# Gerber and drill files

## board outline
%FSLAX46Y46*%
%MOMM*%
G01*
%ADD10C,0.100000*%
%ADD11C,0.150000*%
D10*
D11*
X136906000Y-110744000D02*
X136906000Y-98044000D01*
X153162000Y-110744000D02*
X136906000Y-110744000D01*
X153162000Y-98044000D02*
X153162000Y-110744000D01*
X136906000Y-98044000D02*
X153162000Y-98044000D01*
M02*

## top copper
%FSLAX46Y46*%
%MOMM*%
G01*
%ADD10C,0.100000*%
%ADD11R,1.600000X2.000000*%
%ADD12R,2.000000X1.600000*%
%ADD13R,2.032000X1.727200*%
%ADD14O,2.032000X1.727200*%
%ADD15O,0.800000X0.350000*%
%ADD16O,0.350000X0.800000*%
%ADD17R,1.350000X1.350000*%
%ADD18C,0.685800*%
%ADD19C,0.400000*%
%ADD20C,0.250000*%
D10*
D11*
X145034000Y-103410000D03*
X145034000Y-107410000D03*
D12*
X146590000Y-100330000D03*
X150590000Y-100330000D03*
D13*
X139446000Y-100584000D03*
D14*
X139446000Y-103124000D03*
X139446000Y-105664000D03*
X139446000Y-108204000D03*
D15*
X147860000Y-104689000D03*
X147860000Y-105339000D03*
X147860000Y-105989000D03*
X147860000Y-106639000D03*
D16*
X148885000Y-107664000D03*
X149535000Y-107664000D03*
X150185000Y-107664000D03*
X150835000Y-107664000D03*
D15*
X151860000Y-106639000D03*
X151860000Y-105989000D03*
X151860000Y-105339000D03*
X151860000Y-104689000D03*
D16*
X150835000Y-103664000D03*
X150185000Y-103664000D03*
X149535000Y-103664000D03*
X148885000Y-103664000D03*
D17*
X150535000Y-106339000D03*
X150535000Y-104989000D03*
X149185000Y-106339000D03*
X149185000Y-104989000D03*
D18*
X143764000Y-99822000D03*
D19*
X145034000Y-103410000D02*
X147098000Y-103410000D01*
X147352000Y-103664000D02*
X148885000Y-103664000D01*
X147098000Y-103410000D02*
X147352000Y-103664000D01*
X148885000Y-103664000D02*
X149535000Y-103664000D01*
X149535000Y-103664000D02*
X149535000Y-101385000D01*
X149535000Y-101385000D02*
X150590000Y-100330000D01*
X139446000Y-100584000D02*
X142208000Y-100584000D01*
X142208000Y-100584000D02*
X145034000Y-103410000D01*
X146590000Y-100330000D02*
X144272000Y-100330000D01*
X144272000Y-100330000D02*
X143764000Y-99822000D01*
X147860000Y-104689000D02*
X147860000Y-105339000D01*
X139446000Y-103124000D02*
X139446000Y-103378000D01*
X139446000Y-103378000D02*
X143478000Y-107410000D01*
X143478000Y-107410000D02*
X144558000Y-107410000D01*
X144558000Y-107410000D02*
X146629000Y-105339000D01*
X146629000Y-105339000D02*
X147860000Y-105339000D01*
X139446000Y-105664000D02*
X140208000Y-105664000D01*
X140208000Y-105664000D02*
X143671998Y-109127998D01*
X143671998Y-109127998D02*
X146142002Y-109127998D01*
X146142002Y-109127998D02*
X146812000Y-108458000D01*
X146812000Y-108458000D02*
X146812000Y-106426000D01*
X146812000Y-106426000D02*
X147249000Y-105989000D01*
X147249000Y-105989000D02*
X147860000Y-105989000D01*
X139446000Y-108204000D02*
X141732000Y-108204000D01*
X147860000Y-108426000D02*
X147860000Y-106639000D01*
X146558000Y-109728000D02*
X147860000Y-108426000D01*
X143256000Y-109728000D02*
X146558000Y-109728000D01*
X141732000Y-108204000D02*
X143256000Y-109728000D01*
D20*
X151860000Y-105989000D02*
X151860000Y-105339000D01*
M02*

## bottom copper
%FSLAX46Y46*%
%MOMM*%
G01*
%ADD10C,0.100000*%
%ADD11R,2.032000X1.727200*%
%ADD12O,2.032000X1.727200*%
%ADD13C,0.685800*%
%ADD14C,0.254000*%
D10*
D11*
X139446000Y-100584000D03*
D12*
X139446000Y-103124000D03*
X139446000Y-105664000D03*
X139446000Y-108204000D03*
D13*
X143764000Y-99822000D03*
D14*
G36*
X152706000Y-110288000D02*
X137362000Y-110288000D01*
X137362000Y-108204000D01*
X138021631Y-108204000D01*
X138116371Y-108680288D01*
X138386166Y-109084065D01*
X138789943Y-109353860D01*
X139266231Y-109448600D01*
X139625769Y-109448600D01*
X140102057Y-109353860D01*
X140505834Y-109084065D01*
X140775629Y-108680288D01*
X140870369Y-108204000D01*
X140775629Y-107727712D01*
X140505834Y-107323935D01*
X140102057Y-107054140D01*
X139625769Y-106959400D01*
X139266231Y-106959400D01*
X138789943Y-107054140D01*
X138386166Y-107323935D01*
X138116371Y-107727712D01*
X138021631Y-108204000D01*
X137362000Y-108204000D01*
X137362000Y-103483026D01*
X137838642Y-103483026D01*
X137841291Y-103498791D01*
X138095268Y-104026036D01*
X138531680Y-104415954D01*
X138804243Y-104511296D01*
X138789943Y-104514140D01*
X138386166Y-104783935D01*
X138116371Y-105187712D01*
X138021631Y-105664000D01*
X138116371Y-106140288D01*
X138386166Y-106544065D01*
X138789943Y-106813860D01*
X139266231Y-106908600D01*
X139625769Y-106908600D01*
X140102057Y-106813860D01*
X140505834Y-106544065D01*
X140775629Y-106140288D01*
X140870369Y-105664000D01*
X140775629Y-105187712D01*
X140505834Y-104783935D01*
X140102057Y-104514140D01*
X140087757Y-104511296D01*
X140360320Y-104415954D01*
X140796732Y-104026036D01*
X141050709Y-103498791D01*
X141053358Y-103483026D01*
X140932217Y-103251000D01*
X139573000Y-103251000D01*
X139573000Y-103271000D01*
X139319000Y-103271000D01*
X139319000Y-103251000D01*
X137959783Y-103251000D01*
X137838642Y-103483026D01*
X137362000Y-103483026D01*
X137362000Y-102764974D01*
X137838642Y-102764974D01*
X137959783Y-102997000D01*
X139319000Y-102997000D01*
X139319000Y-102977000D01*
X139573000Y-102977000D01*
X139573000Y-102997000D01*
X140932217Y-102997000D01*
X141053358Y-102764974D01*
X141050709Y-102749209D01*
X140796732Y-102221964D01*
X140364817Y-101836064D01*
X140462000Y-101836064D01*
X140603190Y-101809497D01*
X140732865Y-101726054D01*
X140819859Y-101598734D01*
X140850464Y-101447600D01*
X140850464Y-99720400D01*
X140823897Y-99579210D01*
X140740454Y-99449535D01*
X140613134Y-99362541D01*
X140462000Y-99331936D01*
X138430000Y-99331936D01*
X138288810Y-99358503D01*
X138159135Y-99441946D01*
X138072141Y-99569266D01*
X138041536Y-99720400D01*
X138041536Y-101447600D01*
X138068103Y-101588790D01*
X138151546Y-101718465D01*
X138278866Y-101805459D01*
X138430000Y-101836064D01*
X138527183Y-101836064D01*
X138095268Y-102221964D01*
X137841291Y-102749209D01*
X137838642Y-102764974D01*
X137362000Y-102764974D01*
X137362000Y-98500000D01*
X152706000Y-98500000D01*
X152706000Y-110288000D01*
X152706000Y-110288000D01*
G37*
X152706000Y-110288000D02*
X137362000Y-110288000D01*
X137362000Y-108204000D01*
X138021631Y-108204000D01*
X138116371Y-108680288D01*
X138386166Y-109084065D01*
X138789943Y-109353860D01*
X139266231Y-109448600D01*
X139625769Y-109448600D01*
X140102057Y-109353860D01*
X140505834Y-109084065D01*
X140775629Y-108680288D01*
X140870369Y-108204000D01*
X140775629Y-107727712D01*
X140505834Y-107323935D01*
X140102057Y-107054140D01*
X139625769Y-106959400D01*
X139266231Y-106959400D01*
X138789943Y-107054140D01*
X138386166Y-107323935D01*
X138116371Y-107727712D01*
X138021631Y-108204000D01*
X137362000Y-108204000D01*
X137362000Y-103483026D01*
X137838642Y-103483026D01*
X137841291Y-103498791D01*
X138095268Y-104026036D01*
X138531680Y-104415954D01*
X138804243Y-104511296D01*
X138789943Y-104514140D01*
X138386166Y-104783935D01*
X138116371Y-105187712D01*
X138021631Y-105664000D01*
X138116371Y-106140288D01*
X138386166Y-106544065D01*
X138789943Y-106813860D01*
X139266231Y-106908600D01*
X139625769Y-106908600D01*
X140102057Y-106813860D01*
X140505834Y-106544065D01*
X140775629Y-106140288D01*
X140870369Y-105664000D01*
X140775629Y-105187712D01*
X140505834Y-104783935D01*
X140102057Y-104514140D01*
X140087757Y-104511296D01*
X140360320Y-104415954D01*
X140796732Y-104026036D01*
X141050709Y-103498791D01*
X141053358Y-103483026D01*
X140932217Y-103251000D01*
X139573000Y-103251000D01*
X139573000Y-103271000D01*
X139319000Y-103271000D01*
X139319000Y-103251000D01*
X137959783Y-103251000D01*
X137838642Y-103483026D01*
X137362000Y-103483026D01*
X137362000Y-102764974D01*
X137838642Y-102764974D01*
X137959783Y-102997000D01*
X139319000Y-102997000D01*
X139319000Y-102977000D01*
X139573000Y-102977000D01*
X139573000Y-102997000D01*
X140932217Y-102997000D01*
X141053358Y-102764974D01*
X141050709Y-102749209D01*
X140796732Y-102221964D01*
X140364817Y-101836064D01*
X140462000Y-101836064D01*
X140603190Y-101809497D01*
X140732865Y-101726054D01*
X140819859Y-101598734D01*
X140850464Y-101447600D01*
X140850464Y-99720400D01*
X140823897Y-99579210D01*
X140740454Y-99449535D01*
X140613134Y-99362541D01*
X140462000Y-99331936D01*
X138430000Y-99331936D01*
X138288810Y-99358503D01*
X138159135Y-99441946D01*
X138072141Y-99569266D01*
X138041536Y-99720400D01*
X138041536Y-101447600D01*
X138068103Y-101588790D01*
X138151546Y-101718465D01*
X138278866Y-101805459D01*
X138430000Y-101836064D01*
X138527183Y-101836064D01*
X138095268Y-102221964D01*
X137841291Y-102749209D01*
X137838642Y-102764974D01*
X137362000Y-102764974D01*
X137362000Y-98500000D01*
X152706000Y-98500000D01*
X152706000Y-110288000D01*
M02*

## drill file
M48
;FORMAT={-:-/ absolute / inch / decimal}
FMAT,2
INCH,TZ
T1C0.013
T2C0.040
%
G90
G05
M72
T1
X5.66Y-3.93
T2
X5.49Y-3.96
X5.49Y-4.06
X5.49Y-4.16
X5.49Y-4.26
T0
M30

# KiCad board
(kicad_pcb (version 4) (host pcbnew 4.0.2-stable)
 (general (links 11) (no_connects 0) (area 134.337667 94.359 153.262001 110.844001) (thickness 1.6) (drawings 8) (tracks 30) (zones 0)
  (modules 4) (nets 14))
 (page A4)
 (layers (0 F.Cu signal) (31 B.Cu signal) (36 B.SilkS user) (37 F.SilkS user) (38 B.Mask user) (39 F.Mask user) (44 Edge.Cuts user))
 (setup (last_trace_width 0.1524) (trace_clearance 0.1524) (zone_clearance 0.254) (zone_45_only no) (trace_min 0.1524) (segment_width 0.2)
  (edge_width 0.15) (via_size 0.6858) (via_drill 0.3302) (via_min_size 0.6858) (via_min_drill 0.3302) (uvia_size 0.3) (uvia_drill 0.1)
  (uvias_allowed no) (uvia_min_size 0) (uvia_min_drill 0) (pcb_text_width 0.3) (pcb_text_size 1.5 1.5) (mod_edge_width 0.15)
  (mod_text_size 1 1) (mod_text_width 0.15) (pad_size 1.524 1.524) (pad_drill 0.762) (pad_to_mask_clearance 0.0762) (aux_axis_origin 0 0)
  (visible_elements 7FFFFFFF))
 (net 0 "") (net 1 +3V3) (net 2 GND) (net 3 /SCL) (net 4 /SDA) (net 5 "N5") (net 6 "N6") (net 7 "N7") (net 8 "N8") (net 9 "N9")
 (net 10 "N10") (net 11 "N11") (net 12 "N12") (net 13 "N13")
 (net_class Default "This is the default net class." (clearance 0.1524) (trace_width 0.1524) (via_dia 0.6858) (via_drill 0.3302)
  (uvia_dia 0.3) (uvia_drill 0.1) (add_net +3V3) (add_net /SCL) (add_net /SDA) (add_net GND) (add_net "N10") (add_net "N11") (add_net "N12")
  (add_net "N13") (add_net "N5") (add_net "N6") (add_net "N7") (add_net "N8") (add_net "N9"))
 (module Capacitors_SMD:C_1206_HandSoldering (layer F.Cu) (at 145.034 105.41 270)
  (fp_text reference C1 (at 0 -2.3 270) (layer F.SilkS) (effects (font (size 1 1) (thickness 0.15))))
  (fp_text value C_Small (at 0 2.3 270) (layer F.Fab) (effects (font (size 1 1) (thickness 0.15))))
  (pad 1 smd rect (at -2 0 270) (size 2 1.6) (layers F.Cu F.Mask) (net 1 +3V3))
  (pad 2 smd rect (at 2 0 270) (size 2 1.6) (layers F.Cu F.Mask) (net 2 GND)))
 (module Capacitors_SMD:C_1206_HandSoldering (layer F.Cu) (at 148.59 100.33)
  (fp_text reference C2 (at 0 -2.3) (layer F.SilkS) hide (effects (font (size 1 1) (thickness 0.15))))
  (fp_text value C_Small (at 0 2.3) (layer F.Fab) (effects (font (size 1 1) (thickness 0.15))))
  (pad 1 smd rect (at -2 0) (size 2 1.6) (layers F.Cu F.Mask) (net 2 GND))
  (pad 2 smd rect (at 2 0) (size 2 1.6) (layers F.Cu F.Mask) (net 1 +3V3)))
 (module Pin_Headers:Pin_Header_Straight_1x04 (layer F.Cu) (at 139.446 100.584)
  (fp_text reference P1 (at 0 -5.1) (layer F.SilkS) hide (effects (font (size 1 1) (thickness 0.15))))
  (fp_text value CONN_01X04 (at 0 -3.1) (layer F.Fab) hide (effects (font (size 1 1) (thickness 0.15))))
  (pad 1 thru_hole rect (at 0 0) (size 2.032 1.7272) (drill 1.016) (layers *.Cu *.Mask F.SilkS) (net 1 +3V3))
  (pad 2 thru_hole oval (at 0 2.54) (size 2.032 1.7272) (drill 1.016) (layers *.Cu *.Mask F.SilkS) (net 2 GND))
  (pad 3 thru_hole oval (at 0 5.08) (size 2.032 1.7272) (drill 1.016) (layers *.Cu *.Mask F.SilkS) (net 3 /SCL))
  (pad 4 thru_hole oval (at 0 7.62) (size 2.032 1.7272) (drill 1.016) (layers *.Cu *.Mask F.SilkS) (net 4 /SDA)))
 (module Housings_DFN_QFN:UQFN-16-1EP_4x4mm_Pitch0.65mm (layer F.Cu) (at 149.86 105.664)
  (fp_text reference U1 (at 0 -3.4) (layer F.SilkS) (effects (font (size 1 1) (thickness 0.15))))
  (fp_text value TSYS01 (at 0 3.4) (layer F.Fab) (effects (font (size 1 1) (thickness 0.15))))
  (pad 1 smd oval (at -2 -0.975) (size 0.8 0.35) (layers F.Cu F.Mask) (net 2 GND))
  (pad 2 smd oval (at -2 -0.325) (size 0.8 0.35) (layers F.Cu F.Mask) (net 2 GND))
  (pad 3 smd oval (at -2 0.325) (size 0.8 0.35) (layers F.Cu F.Mask) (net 3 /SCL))
  (pad 4 smd oval (at -2 0.975) (size 0.8 0.35) (layers F.Cu F.Mask) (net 4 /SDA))
  (pad 5 smd oval (at -0.975 2 90) (size 0.8 0.35) (layers F.Cu F.Mask) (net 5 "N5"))
  (pad 6 smd oval (at -0.325 2 90) (size 0.8 0.35) (layers F.Cu F.Mask) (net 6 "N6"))
  (pad 7 smd oval (at 0.325 2 90) (size 0.8 0.35) (layers F.Cu F.Mask) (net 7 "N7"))
  (pad 8 smd oval (at 0.975 2 90) (size 0.8 0.35) (layers F.Cu F.Mask) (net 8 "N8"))
  (pad 9 smd oval (at 2 0.975) (size 0.8 0.35) (layers F.Cu F.Mask) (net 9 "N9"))
  (pad 10 smd oval (at 2 0.325) (size 0.8 0.35) (layers F.Cu F.Mask) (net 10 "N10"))
  (pad 11 smd oval (at 2 -0.325) (size 0.8 0.35) (layers F.Cu F.Mask) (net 10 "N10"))
  (pad 12 smd oval (at 2 -0.975) (size 0.8 0.35) (layers F.Cu F.Mask) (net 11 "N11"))
  (pad 13 smd oval (at 0.975 -2 90) (size 0.8 0.35) (layers F.Cu F.Mask) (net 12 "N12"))
  (pad 14 smd oval (at 0.325 -2 90) (size 0.8 0.35) (layers F.Cu F.Mask) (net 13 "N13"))
  (pad 15 smd oval (at -0.325 -2 90) (size 0.8 0.35) (layers F.Cu F.Mask) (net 1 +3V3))
  (pad 16 smd oval (at -0.975 -2 90) (size 0.8 0.35) (layers F.Cu F.Mask) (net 1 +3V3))
  (pad 17 smd rect (at 0.675 0.675) (size 1.35 1.35) (layers F.Cu F.Mask) (solder_paste_margin_ratio -0.2))
  (pad 17 smd rect (at 0.675 -0.675) (size 1.35 1.35) (layers F.Cu F.Mask) (solder_paste_margin_ratio -0.2))
  (pad 17 smd rect (at -0.675 0.675) (size 1.35 1.35) (layers F.Cu F.Mask) (solder_paste_margin_ratio -0.2))
  (pad 17 smd rect (at -0.675 -0.675) (size 1.35 1.35) (layers F.Cu F.Mask) (solder_paste_margin_ratio -0.2)))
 (gr_line (start 136.906 110.744) (end 136.906 98.044) (angle 90) (layer Edge.Cuts) (width 0.15))
 (gr_line (start 153.162 110.744) (end 136.906 110.744) (angle 90) (layer Edge.Cuts) (width 0.15))
 (gr_line (start 153.162 98.044) (end 153.162 110.744) (angle 90) (layer Edge.Cuts) (width 0.15))
 (gr_line (start 136.906 98.044) (end 153.162 98.044) (angle 90) (layer Edge.Cuts) (width 0.15))
 (segment (start 145.034 103.41) (end 147.098 103.41) (width 0.4) (layer F.Cu) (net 1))
 (segment (start 147.352 103.664) (end 148.885 103.664) (width 0.4) (layer F.Cu) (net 1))
 (segment (start 147.098 103.41) (end 147.352 103.664) (width 0.4) (layer F.Cu) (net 1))
 (segment (start 148.885 103.664) (end 149.535 103.664) (width 0.4) (layer F.Cu) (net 1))
 (segment (start 149.535 103.664) (end 149.535 101.385) (width 0.4) (layer F.Cu) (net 1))
 (segment (start 149.535 101.385) (end 150.59 100.33) (width 0.4) (layer F.Cu) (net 1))
 (segment (start 139.446 100.584) (end 142.208 100.584) (width 0.4) (layer F.Cu) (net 1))
 (segment (start 142.208 100.584) (end 145.034 103.41) (width 0.4) (layer F.Cu) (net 1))
 (segment (start 146.59 100.33) (end 144.272 100.33) (width 0.4) (layer F.Cu) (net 2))
 (via (at 143.764 99.822) (size 0.6858) (drill 0.3302) (layers F.Cu B.Cu) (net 2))
 (segment (start 144.272 100.33) (end 143.764 99.822) (width 0.4) (layer F.Cu) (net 2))
 (segment (start 147.86 104.689) (end 147.86 105.339) (width 0.4) (layer F.Cu) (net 2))
 (segment (start 139.446 103.124) (end 139.446 103.378) (width 0.4) (layer F.Cu) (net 2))
 (segment (start 139.446 103.378) (end 143.478 107.41) (width 0.4) (layer F.Cu) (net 2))
 (segment (start 143.478 107.41) (end 144.558 107.41) (width 0.4) (layer F.Cu) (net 2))
 (segment (start 144.558 107.41) (end 146.629 105.339) (width 0.4) (layer F.Cu) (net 2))
 (segment (start 146.629 105.339) (end 147.86 105.339) (width 0.4) (layer F.Cu) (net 2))
 (segment (start 139.446 105.664) (end 140.208 105.664) (width 0.4) (layer F.Cu) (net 3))
 (segment (start 140.208 105.664) (end 143.671998 109.127998) (width 0.4) (layer F.Cu) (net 3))
 (segment (start 143.671998 109.127998) (end 146.142002 109.127998) (width 0.4) (layer F.Cu) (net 3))
 (segment (start 146.142002 109.127998) (end 146.812 108.458) (width 0.4) (layer F.Cu) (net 3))
 (segment (start 146.812 108.458) (end 146.812 106.426) (width 0.4) (layer F.Cu) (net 3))
 (segment (start 146.812 106.426) (end 147.249 105.989) (width 0.4) (layer F.Cu) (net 3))
 (segment (start 147.249 105.989) (end 147.86 105.989) (width 0.4) (layer F.Cu) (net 3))
 (segment (start 139.446 108.204) (end 141.732 108.204) (width 0.4) (layer F.Cu) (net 4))
 (segment (start 147.86 108.426) (end 147.86 106.639) (width 0.4) (layer F.Cu) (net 4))
 (segment (start 146.558 109.728) (end 147.86 108.426) (width 0.4) (layer F.Cu) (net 4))
 (segment (start 143.256 109.728) (end 146.558 109.728) (width 0.4) (layer F.Cu) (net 4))
 (segment (start 141.732 108.204) (end 143.256 109.728) (width 0.4) (layer F.Cu) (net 4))
 (segment (start 151.86 105.989) (end 151.86 105.339) (width 0.25) (layer F.Cu) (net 10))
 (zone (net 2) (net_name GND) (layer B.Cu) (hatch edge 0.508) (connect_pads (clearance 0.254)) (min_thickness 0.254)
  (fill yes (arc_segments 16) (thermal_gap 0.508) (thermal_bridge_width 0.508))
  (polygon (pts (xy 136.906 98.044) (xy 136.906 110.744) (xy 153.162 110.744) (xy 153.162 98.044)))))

